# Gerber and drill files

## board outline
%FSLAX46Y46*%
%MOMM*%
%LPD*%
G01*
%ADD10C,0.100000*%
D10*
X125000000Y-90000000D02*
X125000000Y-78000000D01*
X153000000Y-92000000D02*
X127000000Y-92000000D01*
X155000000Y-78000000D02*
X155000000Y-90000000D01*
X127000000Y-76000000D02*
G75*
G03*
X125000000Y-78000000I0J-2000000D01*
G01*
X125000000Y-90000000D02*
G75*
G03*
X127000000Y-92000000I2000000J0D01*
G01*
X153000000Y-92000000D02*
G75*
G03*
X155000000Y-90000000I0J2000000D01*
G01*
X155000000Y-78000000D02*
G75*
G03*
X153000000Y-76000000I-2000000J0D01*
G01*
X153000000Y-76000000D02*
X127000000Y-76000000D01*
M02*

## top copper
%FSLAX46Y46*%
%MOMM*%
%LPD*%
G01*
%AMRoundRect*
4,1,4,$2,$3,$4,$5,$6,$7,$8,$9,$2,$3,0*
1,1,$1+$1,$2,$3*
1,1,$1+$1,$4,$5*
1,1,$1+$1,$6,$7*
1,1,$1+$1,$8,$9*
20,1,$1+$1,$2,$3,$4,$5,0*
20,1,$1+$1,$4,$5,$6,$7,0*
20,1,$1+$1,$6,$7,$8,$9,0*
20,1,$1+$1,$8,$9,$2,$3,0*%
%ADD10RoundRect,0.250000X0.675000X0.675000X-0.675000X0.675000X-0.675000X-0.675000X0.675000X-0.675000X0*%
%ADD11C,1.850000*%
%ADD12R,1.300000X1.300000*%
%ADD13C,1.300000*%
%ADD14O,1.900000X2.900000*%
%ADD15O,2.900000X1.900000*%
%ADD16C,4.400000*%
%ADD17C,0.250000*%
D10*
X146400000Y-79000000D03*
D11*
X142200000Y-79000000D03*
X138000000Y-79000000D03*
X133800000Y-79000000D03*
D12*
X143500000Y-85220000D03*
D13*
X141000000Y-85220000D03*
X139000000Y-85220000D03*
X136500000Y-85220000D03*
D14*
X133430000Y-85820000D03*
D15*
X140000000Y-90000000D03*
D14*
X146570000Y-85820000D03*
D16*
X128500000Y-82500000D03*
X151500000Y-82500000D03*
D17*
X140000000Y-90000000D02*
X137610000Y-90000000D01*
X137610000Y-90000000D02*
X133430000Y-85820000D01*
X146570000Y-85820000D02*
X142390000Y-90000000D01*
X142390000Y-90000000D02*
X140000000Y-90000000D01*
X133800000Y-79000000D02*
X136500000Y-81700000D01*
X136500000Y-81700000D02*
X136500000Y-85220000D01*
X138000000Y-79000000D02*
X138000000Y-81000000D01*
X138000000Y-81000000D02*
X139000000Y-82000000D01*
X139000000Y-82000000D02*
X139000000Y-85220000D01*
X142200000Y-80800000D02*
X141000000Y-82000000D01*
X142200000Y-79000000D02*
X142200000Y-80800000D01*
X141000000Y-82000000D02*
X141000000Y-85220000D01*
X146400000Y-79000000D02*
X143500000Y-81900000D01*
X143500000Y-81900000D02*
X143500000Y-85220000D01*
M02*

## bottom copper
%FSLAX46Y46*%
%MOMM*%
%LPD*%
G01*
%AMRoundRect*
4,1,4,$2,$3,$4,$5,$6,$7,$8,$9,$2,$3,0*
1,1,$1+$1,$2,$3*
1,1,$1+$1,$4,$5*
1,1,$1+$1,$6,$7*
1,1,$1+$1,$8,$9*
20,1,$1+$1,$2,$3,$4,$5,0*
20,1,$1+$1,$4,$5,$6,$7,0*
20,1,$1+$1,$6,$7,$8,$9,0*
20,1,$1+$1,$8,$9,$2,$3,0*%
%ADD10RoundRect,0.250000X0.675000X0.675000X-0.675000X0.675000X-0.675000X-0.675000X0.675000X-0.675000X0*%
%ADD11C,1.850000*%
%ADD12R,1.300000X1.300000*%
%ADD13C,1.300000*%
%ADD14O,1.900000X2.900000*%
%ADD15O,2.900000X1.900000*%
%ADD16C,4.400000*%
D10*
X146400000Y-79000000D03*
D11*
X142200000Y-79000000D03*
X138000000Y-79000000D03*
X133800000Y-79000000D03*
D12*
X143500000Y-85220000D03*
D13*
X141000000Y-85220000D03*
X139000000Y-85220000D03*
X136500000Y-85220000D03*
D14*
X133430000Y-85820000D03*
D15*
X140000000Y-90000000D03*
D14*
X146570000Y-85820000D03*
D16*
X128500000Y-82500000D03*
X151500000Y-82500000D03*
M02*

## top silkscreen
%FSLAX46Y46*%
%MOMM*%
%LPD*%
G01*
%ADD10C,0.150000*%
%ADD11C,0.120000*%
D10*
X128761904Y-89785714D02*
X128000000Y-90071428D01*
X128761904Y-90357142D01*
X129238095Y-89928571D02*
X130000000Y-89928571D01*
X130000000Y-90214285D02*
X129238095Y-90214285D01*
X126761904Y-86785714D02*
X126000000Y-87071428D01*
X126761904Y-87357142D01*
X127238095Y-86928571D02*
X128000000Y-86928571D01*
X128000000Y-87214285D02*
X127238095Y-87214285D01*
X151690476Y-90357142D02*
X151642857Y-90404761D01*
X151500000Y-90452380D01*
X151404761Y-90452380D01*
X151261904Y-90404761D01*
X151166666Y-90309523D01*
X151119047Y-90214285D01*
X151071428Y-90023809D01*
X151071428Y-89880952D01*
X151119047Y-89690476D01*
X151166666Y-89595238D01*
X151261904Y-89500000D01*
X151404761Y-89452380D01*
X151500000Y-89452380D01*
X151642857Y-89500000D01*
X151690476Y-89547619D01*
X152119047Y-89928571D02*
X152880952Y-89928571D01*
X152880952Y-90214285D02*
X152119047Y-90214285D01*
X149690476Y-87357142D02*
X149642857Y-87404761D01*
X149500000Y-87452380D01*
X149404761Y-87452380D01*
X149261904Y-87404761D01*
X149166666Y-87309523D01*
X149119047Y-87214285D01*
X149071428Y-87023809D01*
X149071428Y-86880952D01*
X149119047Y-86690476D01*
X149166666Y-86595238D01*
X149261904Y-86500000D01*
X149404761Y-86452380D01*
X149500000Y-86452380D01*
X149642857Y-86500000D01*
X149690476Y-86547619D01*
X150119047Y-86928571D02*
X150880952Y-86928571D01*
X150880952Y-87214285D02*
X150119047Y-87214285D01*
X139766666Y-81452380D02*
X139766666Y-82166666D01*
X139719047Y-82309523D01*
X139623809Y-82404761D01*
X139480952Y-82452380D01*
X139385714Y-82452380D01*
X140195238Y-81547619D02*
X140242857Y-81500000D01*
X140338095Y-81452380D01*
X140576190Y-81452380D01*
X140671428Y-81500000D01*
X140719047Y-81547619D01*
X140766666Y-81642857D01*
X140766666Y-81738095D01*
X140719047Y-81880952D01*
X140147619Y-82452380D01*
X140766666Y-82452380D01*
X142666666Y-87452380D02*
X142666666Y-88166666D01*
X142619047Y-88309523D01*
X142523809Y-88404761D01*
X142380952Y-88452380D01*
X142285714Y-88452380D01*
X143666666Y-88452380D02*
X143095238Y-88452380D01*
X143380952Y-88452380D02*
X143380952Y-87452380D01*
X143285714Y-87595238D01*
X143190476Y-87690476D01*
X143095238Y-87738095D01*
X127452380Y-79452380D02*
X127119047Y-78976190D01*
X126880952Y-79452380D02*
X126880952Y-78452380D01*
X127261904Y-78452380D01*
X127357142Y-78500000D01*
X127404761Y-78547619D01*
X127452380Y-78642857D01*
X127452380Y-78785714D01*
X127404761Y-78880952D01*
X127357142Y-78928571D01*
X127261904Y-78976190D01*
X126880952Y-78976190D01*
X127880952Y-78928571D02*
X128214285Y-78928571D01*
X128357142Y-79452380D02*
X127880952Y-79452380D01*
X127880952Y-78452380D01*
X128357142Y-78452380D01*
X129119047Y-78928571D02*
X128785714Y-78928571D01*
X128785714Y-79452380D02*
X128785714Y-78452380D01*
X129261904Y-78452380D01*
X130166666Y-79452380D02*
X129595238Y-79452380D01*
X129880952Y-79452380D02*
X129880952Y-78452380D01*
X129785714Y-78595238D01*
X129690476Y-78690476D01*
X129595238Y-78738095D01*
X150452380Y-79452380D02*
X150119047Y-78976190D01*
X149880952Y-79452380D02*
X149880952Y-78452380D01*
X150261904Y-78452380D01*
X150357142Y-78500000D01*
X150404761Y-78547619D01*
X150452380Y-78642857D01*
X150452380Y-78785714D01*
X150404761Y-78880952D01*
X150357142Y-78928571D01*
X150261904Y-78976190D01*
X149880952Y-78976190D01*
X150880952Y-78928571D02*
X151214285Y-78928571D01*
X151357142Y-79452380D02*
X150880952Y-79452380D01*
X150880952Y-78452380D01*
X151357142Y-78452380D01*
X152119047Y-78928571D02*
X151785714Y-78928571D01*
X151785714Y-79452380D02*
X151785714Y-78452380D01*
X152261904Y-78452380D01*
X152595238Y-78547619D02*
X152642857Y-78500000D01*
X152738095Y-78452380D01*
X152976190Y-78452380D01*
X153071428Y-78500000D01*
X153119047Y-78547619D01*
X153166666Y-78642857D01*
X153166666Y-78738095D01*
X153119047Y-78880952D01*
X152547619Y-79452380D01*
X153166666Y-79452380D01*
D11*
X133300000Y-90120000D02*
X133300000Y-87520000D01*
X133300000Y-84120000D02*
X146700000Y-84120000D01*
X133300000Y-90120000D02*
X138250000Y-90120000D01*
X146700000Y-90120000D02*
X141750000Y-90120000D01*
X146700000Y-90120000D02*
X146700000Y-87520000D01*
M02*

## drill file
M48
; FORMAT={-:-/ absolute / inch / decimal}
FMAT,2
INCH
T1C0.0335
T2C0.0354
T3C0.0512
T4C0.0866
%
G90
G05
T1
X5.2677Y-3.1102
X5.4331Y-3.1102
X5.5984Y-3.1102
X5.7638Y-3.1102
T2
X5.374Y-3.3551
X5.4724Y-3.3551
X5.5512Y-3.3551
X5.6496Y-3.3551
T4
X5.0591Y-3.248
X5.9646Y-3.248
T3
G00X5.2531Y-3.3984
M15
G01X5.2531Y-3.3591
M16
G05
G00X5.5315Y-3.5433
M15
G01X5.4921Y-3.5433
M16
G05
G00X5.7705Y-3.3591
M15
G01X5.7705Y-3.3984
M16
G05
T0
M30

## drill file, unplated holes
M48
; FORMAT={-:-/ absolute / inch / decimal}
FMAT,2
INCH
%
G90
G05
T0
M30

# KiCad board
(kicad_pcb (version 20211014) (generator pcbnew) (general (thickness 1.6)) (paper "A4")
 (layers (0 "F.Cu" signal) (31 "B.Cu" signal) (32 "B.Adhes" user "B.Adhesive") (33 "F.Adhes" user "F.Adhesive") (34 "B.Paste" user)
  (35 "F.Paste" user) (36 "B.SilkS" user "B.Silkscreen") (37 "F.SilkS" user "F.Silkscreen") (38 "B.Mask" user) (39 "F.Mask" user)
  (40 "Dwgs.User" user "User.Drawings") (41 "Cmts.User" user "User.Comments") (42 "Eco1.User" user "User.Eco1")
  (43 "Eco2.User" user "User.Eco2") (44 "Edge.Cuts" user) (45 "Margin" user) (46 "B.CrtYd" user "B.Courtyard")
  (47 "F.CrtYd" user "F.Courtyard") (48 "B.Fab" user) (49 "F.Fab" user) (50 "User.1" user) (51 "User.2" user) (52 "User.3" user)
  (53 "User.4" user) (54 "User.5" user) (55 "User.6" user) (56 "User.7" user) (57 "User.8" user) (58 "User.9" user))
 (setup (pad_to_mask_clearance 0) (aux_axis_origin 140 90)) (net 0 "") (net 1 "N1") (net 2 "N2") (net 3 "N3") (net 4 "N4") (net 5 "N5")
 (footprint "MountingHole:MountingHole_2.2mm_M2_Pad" (layer "F.Cu") (at 128.5 82.5)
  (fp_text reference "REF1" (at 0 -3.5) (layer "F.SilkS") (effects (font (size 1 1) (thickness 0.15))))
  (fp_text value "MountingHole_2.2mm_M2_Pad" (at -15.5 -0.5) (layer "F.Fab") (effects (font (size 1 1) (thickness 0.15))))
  (pad "1" thru_hole circle (at 0 0) (size 4.4 4.4) (drill 2.2) (layers *.Cu *.Mask)))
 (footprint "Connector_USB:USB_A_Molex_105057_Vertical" (layer "F.Cu") (at 143.5 85.22 180)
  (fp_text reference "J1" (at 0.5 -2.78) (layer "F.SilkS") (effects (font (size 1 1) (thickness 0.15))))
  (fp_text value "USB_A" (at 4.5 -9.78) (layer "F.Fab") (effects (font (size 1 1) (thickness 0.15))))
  (fp_line (start 10.2 -4.9) (end 5.25 -4.9) (layer "F.SilkS") (width 0.12))
  (fp_line (start 10.2 1.1) (end -3.2 1.1) (layer "F.SilkS") (width 0.12))
  (fp_line (start -3.2 -4.9) (end -3.2 -2.3) (layer "F.SilkS") (width 0.12))
  (fp_line (start 10.2 -4.9) (end 10.2 -2.3) (layer "F.SilkS") (width 0.12))
  (fp_line (start -3.2 -4.9) (end 1.75 -4.9) (layer "F.SilkS") (width 0.12))
  (pad "1" thru_hole rect (at 0 0 180) (size 1.3 1.3) (drill 0.9) (layers *.Cu *.Mask) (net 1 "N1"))
  (pad "2" thru_hole circle (at 2.5 0 180) (size 1.3 1.3) (drill 0.9) (layers *.Cu *.Mask) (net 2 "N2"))
  (pad "3" thru_hole circle (at 4.5 0 180) (size 1.3 1.3) (drill 0.9) (layers *.Cu *.Mask) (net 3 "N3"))
  (pad "4" thru_hole circle (at 7 0 180) (size 1.3 1.3) (drill 0.9) (layers *.Cu *.Mask) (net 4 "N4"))
  (pad "5" thru_hole oval (at 10.07 -0.6 180) (size 1.9 2.9) (drill oval 1.3 2.3) (layers *.Cu *.Mask) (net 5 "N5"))
  (pad "5" thru_hole oval (at -3.07 -0.6) (size 1.9 2.9) (drill oval 1.3 2.3) (layers *.Cu *.Mask) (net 5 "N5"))
  (pad "5" thru_hole oval (at 3.5 -4.78 270) (size 1.9 2.9) (drill oval 1.3 2.3) (layers *.Cu *.Mask) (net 5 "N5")))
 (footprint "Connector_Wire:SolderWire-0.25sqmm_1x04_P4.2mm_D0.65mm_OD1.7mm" (layer "F.Cu") (at 146.4 79 180)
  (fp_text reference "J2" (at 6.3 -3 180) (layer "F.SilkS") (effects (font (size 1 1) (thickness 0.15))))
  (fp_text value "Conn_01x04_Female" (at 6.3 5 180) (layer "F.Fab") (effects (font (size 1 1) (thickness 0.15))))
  (pad "1" thru_hole roundrect (at 0 0 180) (size 1.85 1.85) (drill 0.85) (layers *.Cu *.Mask) (roundrect_rratio 0.1351351351) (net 1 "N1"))
  (pad "2" thru_hole circle (at 4.2 0 180) (size 1.85 1.85) (drill 0.85) (layers *.Cu *.Mask) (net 2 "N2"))
  (pad "3" thru_hole circle (at 8.4 0 180) (size 1.85 1.85) (drill 0.85) (layers *.Cu *.Mask) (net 3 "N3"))
  (pad "4" thru_hole circle (at 12.6 0 180) (size 1.85 1.85) (drill 0.85) (layers *.Cu *.Mask) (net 4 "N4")))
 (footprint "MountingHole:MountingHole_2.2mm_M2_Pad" (layer "F.Cu") (at 151.5 82.5)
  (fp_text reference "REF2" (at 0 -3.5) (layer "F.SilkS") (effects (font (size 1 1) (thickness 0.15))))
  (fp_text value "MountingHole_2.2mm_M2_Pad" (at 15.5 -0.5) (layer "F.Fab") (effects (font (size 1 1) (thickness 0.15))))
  (pad "1" thru_hole circle (at 0 0) (size 4.4 4.4) (drill 2.2) (layers *.Cu *.Mask)))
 (gr_arc (start 153 76) (mid 154.414214 76.585786) (end 155 78) (layer "Edge.Cuts") (width 0.1))
 (gr_arc (start 127 92) (mid 125.585786 91.414214) (end 125 90) (layer "Edge.Cuts") (width 0.1))
 (gr_arc (start 155 90) (mid 154.414214 91.414214) (end 153 92) (layer "Edge.Cuts") (width 0.1))
 (gr_line (start 125 90) (end 125 78) (layer "Edge.Cuts") (width 0.1))
 (gr_line (start 153 92) (end 127 92) (layer "Edge.Cuts") (width 0.1))
 (gr_line (start 155 78) (end 155 90) (layer "Edge.Cuts") (width 0.1))
 (gr_line (start 153 76) (end 127 76) (layer "Edge.Cuts") (width 0.1))
 (gr_arc (start 125 78) (mid 125.585786 76.585786) (end 127 76) (layer "Edge.Cuts") (width 0.1))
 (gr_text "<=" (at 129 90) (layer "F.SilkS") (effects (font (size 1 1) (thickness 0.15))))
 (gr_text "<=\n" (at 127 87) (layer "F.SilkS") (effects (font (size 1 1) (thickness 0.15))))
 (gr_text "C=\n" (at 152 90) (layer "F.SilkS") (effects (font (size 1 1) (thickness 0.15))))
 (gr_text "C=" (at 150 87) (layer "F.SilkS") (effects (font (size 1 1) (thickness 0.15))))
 (segment (start 146.4 79) (end 143.5 81.9) (width 0.25) (layer "F.Cu") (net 1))
 (segment (start 143.5 81.9) (end 143.5 85.22) (width 0.25) (layer "F.Cu") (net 1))
 (segment (start 142.2 79) (end 142.2 80.8) (width 0.25) (layer "F.Cu") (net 2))
 (segment (start 142.2 80.8) (end 141 82) (width 0.25) (layer "F.Cu") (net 2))
 (segment (start 141 82) (end 141 85.22) (width 0.25) (layer "F.Cu") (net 2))
 (segment (start 138 79) (end 138 81) (width 0.25) (layer "F.Cu") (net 3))
 (segment (start 139 82) (end 139 85.22) (width 0.25) (layer "F.Cu") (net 3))
 (segment (start 138 81) (end 139 82) (width 0.25) (layer "F.Cu") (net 3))
 (segment (start 133.8 79) (end 136.5 81.7) (width 0.25) (layer "F.Cu") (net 4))
 (segment (start 136.5 81.7) (end 136.5 85.22) (width 0.25) (layer "F.Cu") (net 4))
 (segment (start 142.39 90) (end 140 90) (width 0.25) (layer "F.Cu") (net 5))
 (segment (start 140 90) (end 137.61 90) (width 0.25) (layer "F.Cu") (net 5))
 (segment (start 146.57 85.82) (end 142.39 90) (width 0.25) (layer "F.Cu") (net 5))
 (segment (start 137.61 90) (end 133.43 85.82) (width 0.25) (layer "F.Cu") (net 5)))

